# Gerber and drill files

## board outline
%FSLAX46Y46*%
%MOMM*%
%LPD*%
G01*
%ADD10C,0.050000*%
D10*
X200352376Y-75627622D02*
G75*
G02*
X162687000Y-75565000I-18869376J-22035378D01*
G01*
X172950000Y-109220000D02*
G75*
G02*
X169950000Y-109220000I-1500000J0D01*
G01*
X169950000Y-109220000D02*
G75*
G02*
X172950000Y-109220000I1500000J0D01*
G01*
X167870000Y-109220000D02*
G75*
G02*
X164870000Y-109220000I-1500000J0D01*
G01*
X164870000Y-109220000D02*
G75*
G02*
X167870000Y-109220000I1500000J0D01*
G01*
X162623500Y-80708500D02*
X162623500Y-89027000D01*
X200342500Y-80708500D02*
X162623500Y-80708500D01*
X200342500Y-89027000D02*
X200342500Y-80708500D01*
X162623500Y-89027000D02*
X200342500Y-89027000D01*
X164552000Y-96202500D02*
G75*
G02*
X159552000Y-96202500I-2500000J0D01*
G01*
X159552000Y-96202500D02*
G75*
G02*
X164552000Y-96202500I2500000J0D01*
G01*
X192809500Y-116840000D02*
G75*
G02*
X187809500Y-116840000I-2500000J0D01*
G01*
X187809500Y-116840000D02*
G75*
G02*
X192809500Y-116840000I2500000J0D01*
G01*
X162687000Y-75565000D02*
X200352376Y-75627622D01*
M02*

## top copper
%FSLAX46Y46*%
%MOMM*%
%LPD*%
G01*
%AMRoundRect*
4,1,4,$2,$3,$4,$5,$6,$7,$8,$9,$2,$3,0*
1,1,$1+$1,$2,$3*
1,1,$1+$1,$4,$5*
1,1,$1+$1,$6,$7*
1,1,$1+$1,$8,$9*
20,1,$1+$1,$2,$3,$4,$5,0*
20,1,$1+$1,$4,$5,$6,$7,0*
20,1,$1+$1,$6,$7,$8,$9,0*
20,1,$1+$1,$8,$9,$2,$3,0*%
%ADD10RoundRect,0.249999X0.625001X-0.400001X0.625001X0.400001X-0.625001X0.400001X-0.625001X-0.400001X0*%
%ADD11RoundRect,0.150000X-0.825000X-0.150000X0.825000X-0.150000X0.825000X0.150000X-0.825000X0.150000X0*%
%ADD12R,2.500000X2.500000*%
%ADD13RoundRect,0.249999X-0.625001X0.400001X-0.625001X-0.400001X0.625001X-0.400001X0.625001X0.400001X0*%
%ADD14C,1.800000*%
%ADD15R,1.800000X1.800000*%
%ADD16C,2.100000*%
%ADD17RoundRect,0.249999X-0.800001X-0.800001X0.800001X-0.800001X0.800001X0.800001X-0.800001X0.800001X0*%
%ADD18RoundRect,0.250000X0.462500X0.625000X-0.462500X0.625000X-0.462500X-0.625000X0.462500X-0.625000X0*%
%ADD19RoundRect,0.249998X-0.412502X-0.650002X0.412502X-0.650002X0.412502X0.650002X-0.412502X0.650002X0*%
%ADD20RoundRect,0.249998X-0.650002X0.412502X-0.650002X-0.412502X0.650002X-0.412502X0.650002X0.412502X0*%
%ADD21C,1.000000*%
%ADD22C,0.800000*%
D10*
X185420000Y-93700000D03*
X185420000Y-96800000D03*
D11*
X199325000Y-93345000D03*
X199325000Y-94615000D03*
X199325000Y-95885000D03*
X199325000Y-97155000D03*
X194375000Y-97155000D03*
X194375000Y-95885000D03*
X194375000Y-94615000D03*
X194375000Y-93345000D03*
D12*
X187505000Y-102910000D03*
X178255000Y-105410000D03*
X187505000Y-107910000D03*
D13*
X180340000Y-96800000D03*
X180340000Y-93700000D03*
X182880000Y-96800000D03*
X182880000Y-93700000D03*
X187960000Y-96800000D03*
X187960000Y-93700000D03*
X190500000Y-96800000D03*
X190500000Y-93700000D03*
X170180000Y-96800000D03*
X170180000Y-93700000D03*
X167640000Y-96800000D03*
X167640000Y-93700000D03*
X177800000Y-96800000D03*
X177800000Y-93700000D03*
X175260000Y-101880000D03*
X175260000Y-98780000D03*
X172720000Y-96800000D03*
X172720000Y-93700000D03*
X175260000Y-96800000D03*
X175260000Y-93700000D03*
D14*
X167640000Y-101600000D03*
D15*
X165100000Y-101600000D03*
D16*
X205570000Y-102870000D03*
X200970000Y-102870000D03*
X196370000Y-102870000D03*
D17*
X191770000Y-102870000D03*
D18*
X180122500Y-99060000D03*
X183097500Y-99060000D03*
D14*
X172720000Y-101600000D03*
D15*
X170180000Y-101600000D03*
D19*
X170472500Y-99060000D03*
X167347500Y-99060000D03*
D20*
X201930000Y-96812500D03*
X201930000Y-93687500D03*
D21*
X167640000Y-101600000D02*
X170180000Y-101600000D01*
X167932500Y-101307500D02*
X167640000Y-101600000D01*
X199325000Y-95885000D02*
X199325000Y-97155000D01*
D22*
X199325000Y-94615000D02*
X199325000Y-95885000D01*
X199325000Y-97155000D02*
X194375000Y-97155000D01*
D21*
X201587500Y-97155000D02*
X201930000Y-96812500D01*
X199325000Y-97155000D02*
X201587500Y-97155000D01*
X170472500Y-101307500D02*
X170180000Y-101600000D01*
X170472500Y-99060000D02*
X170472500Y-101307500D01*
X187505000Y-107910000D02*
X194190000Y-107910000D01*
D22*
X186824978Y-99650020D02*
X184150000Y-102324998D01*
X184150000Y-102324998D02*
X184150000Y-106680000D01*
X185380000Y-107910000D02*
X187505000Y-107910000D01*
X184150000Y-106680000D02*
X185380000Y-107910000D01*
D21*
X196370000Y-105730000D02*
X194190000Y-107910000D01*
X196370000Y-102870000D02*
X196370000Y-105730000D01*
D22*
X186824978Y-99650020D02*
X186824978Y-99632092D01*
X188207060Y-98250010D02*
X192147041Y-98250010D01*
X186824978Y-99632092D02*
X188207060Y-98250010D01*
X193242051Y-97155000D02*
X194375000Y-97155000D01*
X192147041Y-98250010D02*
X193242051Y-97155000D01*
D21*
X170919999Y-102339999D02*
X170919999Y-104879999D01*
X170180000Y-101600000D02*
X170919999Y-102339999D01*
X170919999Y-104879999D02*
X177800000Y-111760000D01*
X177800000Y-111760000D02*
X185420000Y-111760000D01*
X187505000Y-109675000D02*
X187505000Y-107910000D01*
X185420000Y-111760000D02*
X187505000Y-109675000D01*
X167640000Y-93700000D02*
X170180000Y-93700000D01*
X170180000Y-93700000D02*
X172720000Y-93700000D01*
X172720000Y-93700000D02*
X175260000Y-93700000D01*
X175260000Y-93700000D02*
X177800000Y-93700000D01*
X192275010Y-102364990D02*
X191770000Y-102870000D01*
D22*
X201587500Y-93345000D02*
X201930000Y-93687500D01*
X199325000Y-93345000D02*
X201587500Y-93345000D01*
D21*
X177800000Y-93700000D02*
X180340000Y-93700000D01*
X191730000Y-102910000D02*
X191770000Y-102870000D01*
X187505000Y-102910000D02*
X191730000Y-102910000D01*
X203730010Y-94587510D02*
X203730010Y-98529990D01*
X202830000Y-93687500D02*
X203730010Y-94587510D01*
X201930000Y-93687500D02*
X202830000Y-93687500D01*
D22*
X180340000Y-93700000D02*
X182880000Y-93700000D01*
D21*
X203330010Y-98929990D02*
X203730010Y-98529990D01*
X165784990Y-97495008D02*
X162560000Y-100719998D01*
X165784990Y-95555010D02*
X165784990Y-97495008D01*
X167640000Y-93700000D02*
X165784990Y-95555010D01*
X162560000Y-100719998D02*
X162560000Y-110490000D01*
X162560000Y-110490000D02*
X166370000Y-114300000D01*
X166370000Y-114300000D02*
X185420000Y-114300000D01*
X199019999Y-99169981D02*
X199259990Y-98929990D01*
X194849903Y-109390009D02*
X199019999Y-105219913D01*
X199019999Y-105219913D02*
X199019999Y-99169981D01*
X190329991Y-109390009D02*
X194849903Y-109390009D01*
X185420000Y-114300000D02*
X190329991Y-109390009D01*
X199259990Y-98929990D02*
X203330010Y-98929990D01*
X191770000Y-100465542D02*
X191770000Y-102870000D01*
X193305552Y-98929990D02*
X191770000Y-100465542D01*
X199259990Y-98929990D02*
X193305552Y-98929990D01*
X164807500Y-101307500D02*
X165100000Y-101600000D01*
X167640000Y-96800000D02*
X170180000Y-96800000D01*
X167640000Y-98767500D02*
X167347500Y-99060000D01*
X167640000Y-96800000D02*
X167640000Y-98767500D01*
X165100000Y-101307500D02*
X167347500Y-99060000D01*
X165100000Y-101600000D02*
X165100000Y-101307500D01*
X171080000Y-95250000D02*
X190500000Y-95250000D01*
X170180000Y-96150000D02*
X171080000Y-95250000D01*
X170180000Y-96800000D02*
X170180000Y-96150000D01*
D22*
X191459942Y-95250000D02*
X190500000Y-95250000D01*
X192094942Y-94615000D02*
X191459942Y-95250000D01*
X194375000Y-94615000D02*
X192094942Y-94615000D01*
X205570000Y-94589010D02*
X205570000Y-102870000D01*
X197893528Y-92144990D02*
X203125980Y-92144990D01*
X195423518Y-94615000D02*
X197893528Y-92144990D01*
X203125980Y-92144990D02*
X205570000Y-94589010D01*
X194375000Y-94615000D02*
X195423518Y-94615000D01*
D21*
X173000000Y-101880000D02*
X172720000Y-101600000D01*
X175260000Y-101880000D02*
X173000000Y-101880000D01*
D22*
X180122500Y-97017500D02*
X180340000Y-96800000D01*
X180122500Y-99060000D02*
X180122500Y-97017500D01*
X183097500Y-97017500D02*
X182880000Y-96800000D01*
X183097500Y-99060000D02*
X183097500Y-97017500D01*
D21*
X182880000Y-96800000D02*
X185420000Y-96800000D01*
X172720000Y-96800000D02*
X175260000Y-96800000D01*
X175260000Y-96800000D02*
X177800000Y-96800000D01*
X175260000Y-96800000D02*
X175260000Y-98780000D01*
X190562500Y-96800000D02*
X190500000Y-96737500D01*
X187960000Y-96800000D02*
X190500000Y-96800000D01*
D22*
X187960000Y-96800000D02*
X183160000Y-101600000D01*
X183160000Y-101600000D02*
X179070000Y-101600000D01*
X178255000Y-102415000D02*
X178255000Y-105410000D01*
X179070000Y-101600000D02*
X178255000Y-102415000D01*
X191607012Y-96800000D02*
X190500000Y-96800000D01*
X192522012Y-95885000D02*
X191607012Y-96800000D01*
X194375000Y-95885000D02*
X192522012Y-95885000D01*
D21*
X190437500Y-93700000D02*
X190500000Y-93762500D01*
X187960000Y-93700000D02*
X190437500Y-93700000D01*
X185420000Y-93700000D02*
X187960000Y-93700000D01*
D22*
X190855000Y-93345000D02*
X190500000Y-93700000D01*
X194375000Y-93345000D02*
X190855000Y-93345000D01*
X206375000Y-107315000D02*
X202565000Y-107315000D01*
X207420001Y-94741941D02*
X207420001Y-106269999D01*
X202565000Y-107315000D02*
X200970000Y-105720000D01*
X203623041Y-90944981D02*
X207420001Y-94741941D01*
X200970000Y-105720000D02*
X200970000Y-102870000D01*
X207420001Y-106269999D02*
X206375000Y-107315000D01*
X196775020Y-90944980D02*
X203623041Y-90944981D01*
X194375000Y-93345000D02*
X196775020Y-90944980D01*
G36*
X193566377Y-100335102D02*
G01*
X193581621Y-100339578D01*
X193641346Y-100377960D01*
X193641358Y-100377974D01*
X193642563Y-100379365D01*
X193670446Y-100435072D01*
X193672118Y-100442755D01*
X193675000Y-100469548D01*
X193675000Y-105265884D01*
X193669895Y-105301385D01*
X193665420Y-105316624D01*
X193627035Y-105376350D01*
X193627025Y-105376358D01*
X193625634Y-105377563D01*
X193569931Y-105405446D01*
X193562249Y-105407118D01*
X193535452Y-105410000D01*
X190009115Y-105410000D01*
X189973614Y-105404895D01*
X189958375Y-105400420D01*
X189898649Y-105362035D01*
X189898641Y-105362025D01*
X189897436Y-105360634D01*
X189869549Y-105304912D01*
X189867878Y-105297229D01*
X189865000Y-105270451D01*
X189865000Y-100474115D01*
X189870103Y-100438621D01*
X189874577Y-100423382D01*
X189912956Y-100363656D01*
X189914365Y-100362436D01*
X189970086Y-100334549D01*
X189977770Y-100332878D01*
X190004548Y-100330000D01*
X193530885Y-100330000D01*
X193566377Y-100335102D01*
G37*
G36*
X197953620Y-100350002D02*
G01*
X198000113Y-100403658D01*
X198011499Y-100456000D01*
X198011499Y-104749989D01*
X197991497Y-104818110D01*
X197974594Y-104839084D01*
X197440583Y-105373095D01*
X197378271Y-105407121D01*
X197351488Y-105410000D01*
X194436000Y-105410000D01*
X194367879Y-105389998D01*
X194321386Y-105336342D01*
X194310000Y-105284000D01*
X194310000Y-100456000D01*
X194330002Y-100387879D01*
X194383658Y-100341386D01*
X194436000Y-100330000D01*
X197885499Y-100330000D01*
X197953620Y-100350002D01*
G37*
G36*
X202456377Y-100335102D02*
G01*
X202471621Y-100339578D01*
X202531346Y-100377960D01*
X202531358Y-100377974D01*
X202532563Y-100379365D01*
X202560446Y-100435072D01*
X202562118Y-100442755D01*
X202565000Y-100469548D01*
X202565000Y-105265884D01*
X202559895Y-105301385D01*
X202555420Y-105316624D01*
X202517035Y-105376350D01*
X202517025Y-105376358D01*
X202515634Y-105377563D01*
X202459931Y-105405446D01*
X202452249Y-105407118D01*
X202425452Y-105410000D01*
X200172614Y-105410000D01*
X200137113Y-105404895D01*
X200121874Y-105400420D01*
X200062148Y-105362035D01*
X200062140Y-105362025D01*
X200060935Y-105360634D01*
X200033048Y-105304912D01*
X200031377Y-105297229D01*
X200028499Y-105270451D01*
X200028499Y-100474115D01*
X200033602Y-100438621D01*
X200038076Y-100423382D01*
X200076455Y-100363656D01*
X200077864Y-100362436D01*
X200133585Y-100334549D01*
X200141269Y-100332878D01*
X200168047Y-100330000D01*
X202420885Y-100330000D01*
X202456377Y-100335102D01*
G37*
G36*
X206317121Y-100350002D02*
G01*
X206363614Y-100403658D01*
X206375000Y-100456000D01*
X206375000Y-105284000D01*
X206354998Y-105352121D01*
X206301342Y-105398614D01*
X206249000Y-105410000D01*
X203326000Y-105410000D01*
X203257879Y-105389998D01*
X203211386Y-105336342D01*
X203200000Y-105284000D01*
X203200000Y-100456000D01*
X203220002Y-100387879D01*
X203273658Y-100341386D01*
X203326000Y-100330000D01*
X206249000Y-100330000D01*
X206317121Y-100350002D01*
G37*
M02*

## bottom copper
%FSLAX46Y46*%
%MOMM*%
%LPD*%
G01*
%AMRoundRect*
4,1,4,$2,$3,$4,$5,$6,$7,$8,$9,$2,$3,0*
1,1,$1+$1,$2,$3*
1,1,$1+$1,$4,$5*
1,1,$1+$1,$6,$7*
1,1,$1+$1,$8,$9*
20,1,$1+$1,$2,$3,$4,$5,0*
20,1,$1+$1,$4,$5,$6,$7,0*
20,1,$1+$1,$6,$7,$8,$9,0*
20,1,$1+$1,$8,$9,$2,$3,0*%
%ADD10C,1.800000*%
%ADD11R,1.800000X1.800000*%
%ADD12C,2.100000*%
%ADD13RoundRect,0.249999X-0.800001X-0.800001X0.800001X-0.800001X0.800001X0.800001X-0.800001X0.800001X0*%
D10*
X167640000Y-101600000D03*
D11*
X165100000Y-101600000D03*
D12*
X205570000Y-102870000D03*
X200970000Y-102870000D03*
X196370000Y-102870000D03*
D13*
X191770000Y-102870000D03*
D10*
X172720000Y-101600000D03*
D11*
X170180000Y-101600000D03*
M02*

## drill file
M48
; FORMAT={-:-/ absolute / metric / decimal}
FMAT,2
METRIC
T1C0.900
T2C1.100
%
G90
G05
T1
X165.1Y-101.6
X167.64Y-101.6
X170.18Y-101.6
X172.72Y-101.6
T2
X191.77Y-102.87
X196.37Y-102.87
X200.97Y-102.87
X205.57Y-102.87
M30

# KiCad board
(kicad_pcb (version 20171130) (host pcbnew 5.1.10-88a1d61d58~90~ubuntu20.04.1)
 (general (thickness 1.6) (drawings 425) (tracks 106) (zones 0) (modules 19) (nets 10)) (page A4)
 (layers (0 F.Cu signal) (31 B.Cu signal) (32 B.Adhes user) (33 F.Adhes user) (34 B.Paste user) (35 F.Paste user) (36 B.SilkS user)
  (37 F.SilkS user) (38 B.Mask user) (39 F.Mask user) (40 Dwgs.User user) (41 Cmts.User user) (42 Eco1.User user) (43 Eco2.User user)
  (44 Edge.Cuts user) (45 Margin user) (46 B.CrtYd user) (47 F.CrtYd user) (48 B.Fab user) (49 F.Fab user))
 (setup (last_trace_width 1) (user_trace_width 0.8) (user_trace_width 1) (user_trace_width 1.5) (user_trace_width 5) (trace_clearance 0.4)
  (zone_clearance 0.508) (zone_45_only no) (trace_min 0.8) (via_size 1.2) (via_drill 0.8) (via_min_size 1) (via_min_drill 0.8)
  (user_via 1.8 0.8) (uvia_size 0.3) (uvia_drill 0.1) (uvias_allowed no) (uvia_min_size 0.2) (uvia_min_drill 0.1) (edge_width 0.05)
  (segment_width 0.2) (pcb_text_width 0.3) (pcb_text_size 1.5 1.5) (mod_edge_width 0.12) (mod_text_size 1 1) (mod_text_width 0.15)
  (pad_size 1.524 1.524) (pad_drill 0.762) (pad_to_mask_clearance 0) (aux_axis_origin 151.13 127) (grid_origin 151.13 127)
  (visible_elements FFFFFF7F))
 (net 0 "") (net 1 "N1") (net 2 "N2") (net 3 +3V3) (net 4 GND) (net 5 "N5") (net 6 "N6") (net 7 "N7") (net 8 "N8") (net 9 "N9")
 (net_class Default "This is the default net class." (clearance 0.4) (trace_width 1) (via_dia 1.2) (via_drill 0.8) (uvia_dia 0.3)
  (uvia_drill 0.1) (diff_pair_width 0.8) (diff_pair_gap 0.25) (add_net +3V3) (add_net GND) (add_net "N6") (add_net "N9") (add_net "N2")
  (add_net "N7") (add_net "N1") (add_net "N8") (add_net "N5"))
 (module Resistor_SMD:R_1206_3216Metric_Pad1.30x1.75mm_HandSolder (layer F.Cu) (at 185.42 95.25 90)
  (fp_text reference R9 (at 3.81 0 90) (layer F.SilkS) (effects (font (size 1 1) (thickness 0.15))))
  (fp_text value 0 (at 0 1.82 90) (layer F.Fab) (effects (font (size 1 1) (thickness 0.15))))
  (pad 2 smd roundrect (at 1.55 0 90) (size 1.3 1.75) (layers F.Cu F.Paste F.Mask) (roundrect_rratio 0.1923069230769231) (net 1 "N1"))
  (pad 1 smd roundrect (at -1.55 0 90) (size 1.3 1.75) (layers F.Cu F.Paste F.Mask) (roundrect_rratio 0.1923069230769231) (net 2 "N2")))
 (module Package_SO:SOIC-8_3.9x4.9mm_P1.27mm (layer F.Cu) (at 196.85 95.25)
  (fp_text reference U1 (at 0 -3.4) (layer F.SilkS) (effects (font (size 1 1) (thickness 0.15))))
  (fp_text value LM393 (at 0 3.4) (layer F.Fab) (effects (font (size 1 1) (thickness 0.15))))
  (pad 8 smd roundrect (at 2.475 -1.905) (size 1.95 0.6) (layers F.Cu F.Paste F.Mask) (roundrect_rratio 0.25) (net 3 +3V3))
  (pad 7 smd roundrect (at 2.475 -0.635) (size 1.95 0.6) (layers F.Cu F.Paste F.Mask) (roundrect_rratio 0.25) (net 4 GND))
  (pad 6 smd roundrect (at 2.475 0.635) (size 1.95 0.6) (layers F.Cu F.Paste F.Mask) (roundrect_rratio 0.25) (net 4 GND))
  (pad 5 smd roundrect (at 2.475 1.905) (size 1.95 0.6) (layers F.Cu F.Paste F.Mask) (roundrect_rratio 0.25) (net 4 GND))
  (pad 4 smd roundrect (at -2.475 1.905) (size 1.95 0.6) (layers F.Cu F.Paste F.Mask) (roundrect_rratio 0.25) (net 4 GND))
  (pad 3 smd roundrect (at -2.475 0.635) (size 1.95 0.6) (layers F.Cu F.Paste F.Mask) (roundrect_rratio 0.25) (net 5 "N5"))
  (pad 2 smd roundrect (at -2.475 -0.635) (size 1.95 0.6) (layers F.Cu F.Paste F.Mask) (roundrect_rratio 0.25) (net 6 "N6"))
  (pad 1 smd roundrect (at -2.475 -1.905) (size 1.95 0.6) (layers F.Cu F.Paste F.Mask) (roundrect_rratio 0.25) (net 1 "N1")))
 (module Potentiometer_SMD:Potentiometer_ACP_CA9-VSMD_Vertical (layer F.Cu) (at 182.88 105.41 180)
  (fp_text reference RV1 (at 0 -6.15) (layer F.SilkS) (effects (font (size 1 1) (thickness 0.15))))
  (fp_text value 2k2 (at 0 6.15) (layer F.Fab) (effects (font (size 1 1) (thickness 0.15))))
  (pad 1 smd rect (at -4.625 2.5 180) (size 2.5 2.5) (layers F.Cu F.Paste F.Mask) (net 3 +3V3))
  (pad 2 smd rect (at 4.625 0 180) (size 2.5 2.5) (layers F.Cu F.Paste F.Mask) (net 5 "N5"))
  (pad 3 smd rect (at -4.625 -2.5 180) (size 2.5 2.5) (layers F.Cu F.Paste F.Mask) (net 4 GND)))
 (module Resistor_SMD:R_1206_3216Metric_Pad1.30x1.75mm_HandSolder (layer F.Cu) (at 180.34 95.25 270)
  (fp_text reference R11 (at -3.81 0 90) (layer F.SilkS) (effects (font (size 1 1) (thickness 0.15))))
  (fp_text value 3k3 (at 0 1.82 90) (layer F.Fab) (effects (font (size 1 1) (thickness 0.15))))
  (pad 2 smd roundrect (at 1.55 0 270) (size 1.3 1.75) (layers F.Cu F.Paste F.Mask) (roundrect_rratio 0.1923069230769231) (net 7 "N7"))
  (pad 1 smd roundrect (at -1.55 0 270) (size 1.3 1.75) (layers F.Cu F.Paste F.Mask) (roundrect_rratio 0.1923069230769231) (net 3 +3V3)))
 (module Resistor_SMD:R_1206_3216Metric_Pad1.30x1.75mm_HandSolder (layer F.Cu) (at 182.88 95.25 270)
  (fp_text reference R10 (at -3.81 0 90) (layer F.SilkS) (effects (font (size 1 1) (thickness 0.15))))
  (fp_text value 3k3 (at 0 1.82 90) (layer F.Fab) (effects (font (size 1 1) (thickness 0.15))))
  (pad 2 smd roundrect (at 1.55 0 270) (size 1.3 1.75) (layers F.Cu F.Paste F.Mask) (roundrect_rratio 0.1923069230769231) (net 2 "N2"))
  (pad 1 smd roundrect (at -1.55 0 270) (size 1.3 1.75) (layers F.Cu F.Paste F.Mask) (roundrect_rratio 0.1923069230769231) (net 3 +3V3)))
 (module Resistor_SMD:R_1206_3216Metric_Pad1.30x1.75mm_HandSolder (layer F.Cu) (at 187.96 95.25 270)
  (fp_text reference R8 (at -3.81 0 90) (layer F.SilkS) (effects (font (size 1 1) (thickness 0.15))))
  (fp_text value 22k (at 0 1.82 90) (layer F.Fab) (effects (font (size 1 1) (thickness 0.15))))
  (pad 2 smd roundrect (at 1.55 0 270) (size 1.3 1.75) (layers F.Cu F.Paste F.Mask) (roundrect_rratio 0.1923069230769231) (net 5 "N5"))
  (pad 1 smd roundrect (at -1.55 0 270) (size 1.3 1.75) (layers F.Cu F.Paste F.Mask) (roundrect_rratio 0.1923069230769231) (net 1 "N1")))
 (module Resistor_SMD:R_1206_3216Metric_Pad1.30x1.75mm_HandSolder (layer F.Cu) (at 190.5 95.25 270)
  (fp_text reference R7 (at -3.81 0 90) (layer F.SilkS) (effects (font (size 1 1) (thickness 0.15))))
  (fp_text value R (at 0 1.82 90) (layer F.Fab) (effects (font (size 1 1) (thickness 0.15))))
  (pad 2 smd roundrect (at 1.55 0 270) (size 1.3 1.75) (layers F.Cu F.Paste F.Mask) (roundrect_rratio 0.1923069230769231) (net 5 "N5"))
  (pad 1 smd roundrect (at -1.55 0 270) (size 1.3 1.75) (layers F.Cu F.Paste F.Mask) (roundrect_rratio 0.1923069230769231) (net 1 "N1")))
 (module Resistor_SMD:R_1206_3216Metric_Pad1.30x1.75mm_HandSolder (layer F.Cu) (at 170.18 95.25 270)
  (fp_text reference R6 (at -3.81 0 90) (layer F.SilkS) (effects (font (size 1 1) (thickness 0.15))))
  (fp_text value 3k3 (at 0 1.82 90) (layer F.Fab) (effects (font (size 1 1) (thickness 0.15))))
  (pad 2 smd roundrect (at 1.55 0 270) (size 1.3 1.75) (layers F.Cu F.Paste F.Mask) (roundrect_rratio 0.1923069230769231) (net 6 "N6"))
  (pad 1 smd roundrect (at -1.55 0 270) (size 1.3 1.75) (layers F.Cu F.Paste F.Mask) (roundrect_rratio 0.1923069230769231) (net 3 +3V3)))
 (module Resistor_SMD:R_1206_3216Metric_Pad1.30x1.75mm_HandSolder (layer F.Cu) (at 167.64 95.25 270)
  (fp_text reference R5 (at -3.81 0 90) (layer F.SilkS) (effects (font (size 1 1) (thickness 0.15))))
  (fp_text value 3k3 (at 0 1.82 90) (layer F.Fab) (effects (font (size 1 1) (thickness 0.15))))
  (pad 2 smd roundrect (at 1.55 0 270) (size 1.3 1.75) (layers F.Cu F.Paste F.Mask) (roundrect_rratio 0.1923069230769231) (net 6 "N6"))
  (pad 1 smd roundrect (at -1.55 0 270) (size 1.3 1.75) (layers F.Cu F.Paste F.Mask) (roundrect_rratio 0.1923069230769231) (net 3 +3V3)))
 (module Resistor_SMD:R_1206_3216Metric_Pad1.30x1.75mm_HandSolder (layer F.Cu) (at 177.8 95.25 270)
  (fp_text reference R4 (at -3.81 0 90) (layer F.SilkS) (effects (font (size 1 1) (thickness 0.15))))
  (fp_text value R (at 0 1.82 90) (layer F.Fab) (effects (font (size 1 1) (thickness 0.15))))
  (pad 2 smd roundrect (at 1.55 0 270) (size 1.3 1.75) (layers F.Cu F.Paste F.Mask) (roundrect_rratio 0.1923069230769231) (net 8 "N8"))
  (pad 1 smd roundrect (at -1.55 0 270) (size 1.3 1.75) (layers F.Cu F.Paste F.Mask) (roundrect_rratio 0.1923069230769231) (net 3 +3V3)))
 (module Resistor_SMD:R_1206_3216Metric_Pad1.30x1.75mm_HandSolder (layer F.Cu) (at 175.26 100.33 270)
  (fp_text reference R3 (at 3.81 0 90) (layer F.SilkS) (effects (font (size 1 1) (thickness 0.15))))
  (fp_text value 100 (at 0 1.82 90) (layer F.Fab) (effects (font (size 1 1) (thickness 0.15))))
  (pad 2 smd roundrect (at 1.55 0 270) (size 1.3 1.75) (layers F.Cu F.Paste F.Mask) (roundrect_rratio 0.1923069230769231) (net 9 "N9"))
  (pad 1 smd roundrect (at -1.55 0 270) (size 1.3 1.75) (layers F.Cu F.Paste F.Mask) (roundrect_rratio 0.1923069230769231) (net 8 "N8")))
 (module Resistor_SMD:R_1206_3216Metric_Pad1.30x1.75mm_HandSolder (layer F.Cu) (at 172.72 95.25 270)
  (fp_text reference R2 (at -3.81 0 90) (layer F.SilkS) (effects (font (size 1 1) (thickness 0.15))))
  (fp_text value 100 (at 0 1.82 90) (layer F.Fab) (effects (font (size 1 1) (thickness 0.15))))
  (pad 2 smd roundrect (at 1.55 0 270) (size 1.3 1.75) (layers F.Cu F.Paste F.Mask) (roundrect_rratio 0.1923069230769231) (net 8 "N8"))
  (pad 1 smd roundrect (at -1.55 0 270) (size 1.3 1.75) (layers F.Cu F.Paste F.Mask) (roundrect_rratio 0.1923069230769231) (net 3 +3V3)))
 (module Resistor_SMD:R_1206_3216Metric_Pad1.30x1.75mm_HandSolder (layer F.Cu) (at 175.26 95.25 270)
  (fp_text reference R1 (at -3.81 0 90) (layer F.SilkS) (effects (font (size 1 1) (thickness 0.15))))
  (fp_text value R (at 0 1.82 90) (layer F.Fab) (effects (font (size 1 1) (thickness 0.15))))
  (pad 2 smd roundrect (at 1.55 0 270) (size 1.3 1.75) (layers F.Cu F.Paste F.Mask) (roundrect_rratio 0.1923069230769231) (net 8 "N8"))
  (pad 1 smd roundrect (at -1.55 0 270) (size 1.3 1.75) (layers F.Cu F.Paste F.Mask) (roundrect_rratio 0.1923069230769231) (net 3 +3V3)))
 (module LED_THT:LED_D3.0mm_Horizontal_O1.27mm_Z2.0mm (layer F.Cu) (at 165.1 101.6)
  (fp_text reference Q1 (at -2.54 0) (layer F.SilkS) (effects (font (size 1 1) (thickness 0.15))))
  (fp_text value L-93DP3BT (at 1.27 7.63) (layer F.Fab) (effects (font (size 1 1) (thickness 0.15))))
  (pad 2 thru_hole circle (at 2.54 0) (size 1.8 1.8) (drill 0.9) (layers *.Cu *.Mask) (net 4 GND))
  (pad 1 thru_hole rect (at 0 0) (size 1.8 1.8) (drill 0.9) (layers *.Cu *.Mask) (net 6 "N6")))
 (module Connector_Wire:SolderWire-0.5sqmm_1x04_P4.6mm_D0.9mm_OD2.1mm (layer F.Cu) (at 191.77 102.87)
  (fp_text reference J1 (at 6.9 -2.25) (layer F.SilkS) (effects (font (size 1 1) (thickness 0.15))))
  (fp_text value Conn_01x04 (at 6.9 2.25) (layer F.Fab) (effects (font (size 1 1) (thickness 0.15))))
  (pad 4 thru_hole circle (at 13.8 0) (size 2.1 2.1) (drill 1.1) (layers *.Cu *.Mask) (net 6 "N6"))
  (pad 3 thru_hole circle (at 9.2 0) (size 2.1 2.1) (drill 1.1) (layers *.Cu *.Mask) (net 1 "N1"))
  (pad 2 thru_hole circle (at 4.6 0) (size 2.1 2.1) (drill 1.1) (layers *.Cu *.Mask) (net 4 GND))
  (pad 1 thru_hole roundrect (at 0 0) (size 2.1 2.1) (drill 1.1) (layers *.Cu *.Mask) (roundrect_rratio 0.1190471428571429) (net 3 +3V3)))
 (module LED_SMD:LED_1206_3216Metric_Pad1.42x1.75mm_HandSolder (layer F.Cu) (at 181.61 99.06 180)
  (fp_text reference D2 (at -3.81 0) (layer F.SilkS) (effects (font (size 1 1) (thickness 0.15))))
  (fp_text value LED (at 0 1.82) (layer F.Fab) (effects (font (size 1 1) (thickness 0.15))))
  (pad 2 smd roundrect (at 1.4875 0 180) (size 1.425 1.75) (layers F.Cu F.Paste F.Mask) (roundrect_rratio 0.1754385964912281) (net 7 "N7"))
  (pad 1 smd roundrect (at -1.4875 0 180) (size 1.425 1.75) (layers F.Cu F.Paste F.Mask) (roundrect_rratio 0.1754385964912281) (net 2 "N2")))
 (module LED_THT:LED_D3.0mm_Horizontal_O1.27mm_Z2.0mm (layer F.Cu) (at 170.18 101.6)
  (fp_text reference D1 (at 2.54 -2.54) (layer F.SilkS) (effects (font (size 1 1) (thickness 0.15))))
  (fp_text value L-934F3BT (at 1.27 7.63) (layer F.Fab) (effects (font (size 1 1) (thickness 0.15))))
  (pad 2 thru_hole circle (at 2.54 0) (size 1.8 1.8) (drill 0.9) (layers *.Cu *.Mask) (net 9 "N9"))
  (pad 1 thru_hole rect (at 0 0) (size 1.8 1.8) (drill 0.9) (layers *.Cu *.Mask) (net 4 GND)))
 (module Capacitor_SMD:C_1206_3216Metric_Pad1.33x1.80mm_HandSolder (layer F.Cu) (at 168.91 99.06)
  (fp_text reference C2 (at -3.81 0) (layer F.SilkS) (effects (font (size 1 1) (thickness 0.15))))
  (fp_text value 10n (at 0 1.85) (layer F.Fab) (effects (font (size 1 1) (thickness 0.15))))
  (pad 2 smd roundrect (at 1.5625 0) (size 1.325 1.8) (layers F.Cu F.Paste F.Mask) (roundrect_rratio 0.1886777358490566) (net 4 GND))
  (pad 1 smd roundrect (at -1.5625 0) (size 1.325 1.8) (layers F.Cu F.Paste F.Mask) (roundrect_rratio 0.1886777358490566) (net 6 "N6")))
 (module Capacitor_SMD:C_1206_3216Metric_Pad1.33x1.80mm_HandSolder (layer F.Cu) (at 201.93 95.25 270)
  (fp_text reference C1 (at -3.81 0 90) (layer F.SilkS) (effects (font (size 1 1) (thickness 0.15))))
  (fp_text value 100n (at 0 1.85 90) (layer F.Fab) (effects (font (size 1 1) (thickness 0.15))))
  (pad 2 smd roundrect (at 1.5625 0 270) (size 1.325 1.8) (layers F.Cu F.Paste F.Mask) (roundrect_rratio 0.1886777358490566) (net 4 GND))
  (pad 1 smd roundrect (at -1.5625 0 270) (size 1.325 1.8) (layers F.Cu F.Paste F.Mask) (roundrect_rratio 0.1886777358490566) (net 3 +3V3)))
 (gr_arc (start 181.483 97.663) (end 162.687 75.565) (angle -279.0421861) (layer Edge.Cuts) (width 0.05))
 (gr_circle (center 171.45 109.22) (end 172.95 109.22) (layer Edge.Cuts) (width 0.05))
 (gr_circle (center 166.37 109.22) (end 167.87 109.22) (layer Edge.Cuts) (width 0.05))
 (gr_line (start 162.6235 80.7085) (end 162.6235 89.027) (layer Edge.Cuts) (width 0.05))
 (gr_line (start 200.3425 80.7085) (end 162.6235 80.7085) (layer Edge.Cuts) (width 0.05))
 (gr_line (start 200.3425 89.027) (end 200.3425 80.7085) (layer Edge.Cuts) (width 0.05))
 (gr_line (start 162.6235 89.027) (end 200.3425 89.027) (layer Edge.Cuts) (width 0.05))
 (gr_circle (center 162.052 96.2025) (end 164.552 96.2025) (layer Edge.Cuts) (width 0.05))
 (gr_circle (center 190.3095 116.84) (end 192.8095 116.84) (layer Edge.Cuts) (width 0.05))
 (gr_line (start 162.687 75.565) (end 200.352376 75.627622) (layer Edge.Cuts) (width 0.05))
 (segment (start 167.64 101.6) (end 170.18 101.6) (width 1) (layer F.Cu) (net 4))
 (segment (start 167.9325 101.3075) (end 167.64 101.6) (width 1) (layer F.Cu) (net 4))
 (segment (start 199.325 95.885) (end 199.325 97.155) (width 1) (layer F.Cu) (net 4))
 (segment (start 199.325 94.615) (end 199.325 95.885) (width 0.8) (layer F.Cu) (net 4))
 (segment (start 199.325 97.155) (end 194.375 97.155) (width 0.8) (layer F.Cu) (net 4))
 (segment (start 201.5875 97.155) (end 201.93 96.8125) (width 1) (layer F.Cu) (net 4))
 (segment (start 199.325 97.155) (end 201.5875 97.155) (width 1) (layer F.Cu) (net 4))
 (segment (start 170.4725 101.3075) (end 170.18 101.6) (width 1) (layer F.Cu) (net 4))
 (segment (start 170.4725 99.06) (end 170.4725 101.3075) (width 1) (layer F.Cu) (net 4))
 (segment (start 187.505 107.91) (end 194.19 107.91) (width 1) (layer F.Cu) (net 4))
 (segment (start 186.824978 99.65002) (end 184.15 102.324998) (width 0.8) (layer F.Cu) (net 4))
 (segment (start 184.15 102.324998) (end 184.15 106.68) (width 0.8) (layer F.Cu) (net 4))
 (segment (start 185.38 107.91) (end 187.505 107.91) (width 0.8) (layer F.Cu) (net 4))
 (segment (start 184.15 106.68) (end 185.38 107.91) (width 0.8) (layer F.Cu) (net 4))
 (segment (start 196.37 105.73) (end 194.19 107.91) (width 1) (layer F.Cu) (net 4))
 (segment (start 196.37 102.87) (end 196.37 105.73) (width 1) (layer F.Cu) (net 4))
 (segment (start 186.824978 99.65002) (end 186.824978 99.632092) (width 0.8) (layer F.Cu) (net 4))
 (segment (start 188.20706 98.25001) (end 192.147041 98.25001) (width 0.8) (layer F.Cu) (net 4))
 (segment (start 186.824978 99.632092) (end 188.20706 98.25001) (width 0.8) (layer F.Cu) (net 4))
 (segment (start 193.242051 97.155) (end 194.375 97.155) (width 0.8) (layer F.Cu) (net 4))
 (segment (start 192.147041 98.25001) (end 193.242051 97.155) (width 0.8) (layer F.Cu) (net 4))
 (segment (start 170.919999 102.339999) (end 170.919999 104.879999) (width 1) (layer F.Cu) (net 4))
 (segment (start 170.18 101.6) (end 170.919999 102.339999) (width 1) (layer F.Cu) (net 4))
 (segment (start 170.919999 104.879999) (end 177.8 111.76) (width 1) (layer F.Cu) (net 4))
 (segment (start 177.8 111.76) (end 185.42 111.76) (width 1) (layer F.Cu) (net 4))
 (segment (start 187.505 109.675) (end 187.505 107.91) (width 1) (layer F.Cu) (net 4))
 (segment (start 185.42 111.76) (end 187.505 109.675) (width 1) (layer F.Cu) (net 4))
 (segment (start 167.64 93.7) (end 170.18 93.7) (width 1) (layer F.Cu) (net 3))
 (segment (start 170.18 93.7) (end 172.72 93.7) (width 1) (layer F.Cu) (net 3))
 (segment (start 172.72 93.7) (end 175.26 93.7) (width 1) (layer F.Cu) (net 3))
 (segment (start 175.26 93.7) (end 177.8 93.7) (width 1) (layer F.Cu) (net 3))
 (segment (start 192.27501 102.36499) (end 191.77 102.87) (width 1) (layer F.Cu) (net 3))
 (segment (start 201.5875 93.345) (end 201.93 93.6875) (width 0.8) (layer F.Cu) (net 3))
 (segment (start 199.325 93.345) (end 201.5875 93.345) (width 0.8) (layer F.Cu) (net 3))
 (segment (start 177.8 93.7) (end 180.34 93.7) (width 1) (layer F.Cu) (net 3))
 (segment (start 191.73 102.91) (end 191.77 102.87) (width 1) (layer F.Cu) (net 3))
 (segment (start 187.505 102.91) (end 191.73 102.91) (width 1) (layer F.Cu) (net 3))
 (segment (start 203.73001 94.58751) (end 203.73001 98.52999) (width 1) (layer F.Cu) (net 3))
 (segment (start 202.83 93.6875) (end 203.73001 94.58751) (width 1) (layer F.Cu) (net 3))
 (segment (start 201.93 93.6875) (end 202.83 93.6875) (width 1) (layer F.Cu) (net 3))
 (segment (start 180.34 93.7) (end 182.88 93.7) (width 0.8) (layer F.Cu) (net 3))
 (segment (start 203.33001 98.92999) (end 203.73001 98.52999) (width 1) (layer F.Cu) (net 3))
 (segment (start 165.78499 97.495008) (end 162.56 100.719998) (width 1) (layer F.Cu) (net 3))
 (segment (start 165.78499 95.55501) (end 165.78499 97.495008) (width 1) (layer F.Cu) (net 3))
 (segment (start 167.64 93.7) (end 165.78499 95.55501) (width 1) (layer F.Cu) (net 3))
 (segment (start 162.56 100.719998) (end 162.56 110.49) (width 1) (layer F.Cu) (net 3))
 (segment (start 162.56 110.49) (end 166.37 114.3) (width 1) (layer F.Cu) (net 3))
 (segment (start 166.37 114.3) (end 185.42 114.3) (width 1) (layer F.Cu) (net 3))
 (segment (start 199.019999 99.169981) (end 199.25999 98.92999) (width 1) (layer F.Cu) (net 3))
 (segment (start 194.849903 109.390009) (end 199.019999 105.219913) (width 1) (layer F.Cu) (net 3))
 (segment (start 199.019999 105.219913) (end 199.019999 99.169981) (width 1) (layer F.Cu) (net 3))
 (segment (start 190.329991 109.390009) (end 194.849903 109.390009) (width 1) (layer F.Cu) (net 3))
 (segment (start 185.42 114.3) (end 190.329991 109.390009) (width 1) (layer F.Cu) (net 3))
 (segment (start 199.25999 98.92999) (end 203.33001 98.92999) (width 1) (layer F.Cu) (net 3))
 (segment (start 191.77 100.465542) (end 191.77 102.87) (width 1) (layer F.Cu) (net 3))
 (segment (start 193.305552 98.92999) (end 191.77 100.465542) (width 1) (layer F.Cu) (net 3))
 (segment (start 199.25999 98.92999) (end 193.305552 98.92999) (width 1) (layer F.Cu) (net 3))
 (segment (start 164.8075 101.3075) (end 165.1 101.6) (width 1) (layer F.Cu) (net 6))
 (segment (start 167.64 96.8) (end 170.18 96.8) (width 1) (layer F.Cu) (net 6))
 (segment (start 167.64 98.7675) (end 167.3475 99.06) (width 1) (layer F.Cu) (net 6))
 (segment (start 167.64 96.8) (end 167.64 98.7675) (width 1) (layer F.Cu) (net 6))
 (segment (start 165.1 101.3075) (end 167.3475 99.06) (width 1) (layer F.Cu) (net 6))
 (segment (start 165.1 101.6) (end 165.1 101.3075) (width 1) (layer F.Cu) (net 6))
 (segment (start 171.08 95.25) (end 190.5 95.25) (width 1) (layer F.Cu) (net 6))
 (segment (start 170.18 96.15) (end 171.08 95.25) (width 1) (layer F.Cu) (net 6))
 (segment (start 170.18 96.8) (end 170.18 96.15) (width 1) (layer F.Cu) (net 6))
 (segment (start 191.459942 95.25) (end 190.5 95.25) (width 0.8) (layer F.Cu) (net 6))
 (segment (start 192.094942 94.615) (end 191.459942 95.25) (width 0.8) (layer F.Cu) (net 6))
 (segment (start 194.375 94.615) (end 192.094942 94.615) (width 0.8) (layer F.Cu) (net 6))
 (segment (start 205.57 94.58901) (end 205.57 102.87) (width 0.8) (layer F.Cu) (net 6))
 (segment (start 197.893528 92.14499) (end 203.12598 92.14499) (width 0.8) (layer F.Cu) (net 6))
 (segment (start 195.423518 94.615) (end 197.893528 92.14499) (width 0.8) (layer F.Cu) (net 6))
 (segment (start 203.12598 92.14499) (end 205.57 94.58901) (width 0.8) (layer F.Cu) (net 6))
 (segment (start 194.375 94.615) (end 195.423518 94.615) (width 0.8) (layer F.Cu) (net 6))
 (segment (start 173 101.88) (end 172.72 101.6) (width 1) (layer F.Cu) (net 9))
 (segment (start 175.26 101.88) (end 173 101.88) (width 1) (layer F.Cu) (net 9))
 (segment (start 180.1225 97.0175) (end 180.34 96.8) (width 0.8) (layer F.Cu) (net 7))
 (segment (start 180.1225 99.06) (end 180.1225 97.0175) (width 0.8) (layer F.Cu) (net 7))
 (segment (start 183.0975 97.0175) (end 182.88 96.8) (width 0.8) (layer F.Cu) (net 2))
 (segment (start 183.0975 99.06) (end 183.0975 97.0175) (width 0.8) (layer F.Cu) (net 2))
 (segment (start 182.88 96.8) (end 185.42 96.8) (width 1) (layer F.Cu) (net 2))
 (segment (start 172.72 96.8) (end 175.26 96.8) (width 1) (layer F.Cu) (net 8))
 (segment (start 175.26 96.8) (end 177.8 96.8) (width 1) (layer F.Cu) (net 8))
 (segment (start 175.26 96.8) (end 175.26 98.78) (width 1) (layer F.Cu) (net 8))
 (segment (start 190.5625 96.8) (end 190.5 96.7375) (width 1) (layer F.Cu) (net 5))
 (segment (start 187.96 96.8) (end 190.5 96.8) (width 1) (layer F.Cu) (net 5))
 (segment (start 187.96 96.8) (end 183.16 101.6) (width 0.8) (layer F.Cu) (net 5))
 (segment (start 183.16 101.6) (end 179.07 101.6) (width 0.8) (layer F.Cu) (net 5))
 (segment (start 178.255 102.415) (end 178.255 105.41) (width 0.8) (layer F.Cu) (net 5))
 (segment (start 179.07 101.6) (end 178.255 102.415) (width 0.8) (layer F.Cu) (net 5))
 (segment (start 191.607012 96.8) (end 190.5 96.8) (width 0.8) (layer F.Cu) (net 5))
 (segment (start 192.522012 95.885) (end 191.607012 96.8) (width 0.8) (layer F.Cu) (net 5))
 (segment (start 194.375 95.885) (end 192.522012 95.885) (width 0.8) (layer F.Cu) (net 5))
 (segment (start 190.4375 93.7) (end 190.5 93.7625) (width 1) (layer F.Cu) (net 1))
 (segment (start 187.96 93.7) (end 190.4375 93.7) (width 1) (layer F.Cu) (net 1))
 (segment (start 185.42 93.7) (end 187.96 93.7) (width 1) (layer F.Cu) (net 1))
 (segment (start 190.855 93.345) (end 190.5 93.7) (width 0.8) (layer F.Cu) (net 1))
 (segment (start 194.375 93.345) (end 190.855 93.345) (width 0.8) (layer F.Cu) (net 1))
 (segment (start 206.375 107.315) (end 202.565 107.315) (width 0.8) (layer F.Cu) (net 1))
 (segment (start 207.420001 94.741941) (end 207.420001 106.269999) (width 0.8) (layer F.Cu) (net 1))
 (segment (start 202.565 107.315) (end 200.97 105.72) (width 0.8) (layer F.Cu) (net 1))
 (segment (start 203.623041 90.944981) (end 207.420001 94.741941) (width 0.8) (layer F.Cu) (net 1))
 (segment (start 200.97 105.72) (end 200.97 102.87) (width 0.8) (layer F.Cu) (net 1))
 (segment (start 207.420001 106.269999) (end 206.375 107.315) (width 0.8) (layer F.Cu) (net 1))
 (segment (start 196.77502 90.94498) (end 203.623041 90.944981) (width 0.8) (layer F.Cu) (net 1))
 (segment (start 194.375 93.345) (end 196.77502 90.94498) (width 0.8) (layer F.Cu) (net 1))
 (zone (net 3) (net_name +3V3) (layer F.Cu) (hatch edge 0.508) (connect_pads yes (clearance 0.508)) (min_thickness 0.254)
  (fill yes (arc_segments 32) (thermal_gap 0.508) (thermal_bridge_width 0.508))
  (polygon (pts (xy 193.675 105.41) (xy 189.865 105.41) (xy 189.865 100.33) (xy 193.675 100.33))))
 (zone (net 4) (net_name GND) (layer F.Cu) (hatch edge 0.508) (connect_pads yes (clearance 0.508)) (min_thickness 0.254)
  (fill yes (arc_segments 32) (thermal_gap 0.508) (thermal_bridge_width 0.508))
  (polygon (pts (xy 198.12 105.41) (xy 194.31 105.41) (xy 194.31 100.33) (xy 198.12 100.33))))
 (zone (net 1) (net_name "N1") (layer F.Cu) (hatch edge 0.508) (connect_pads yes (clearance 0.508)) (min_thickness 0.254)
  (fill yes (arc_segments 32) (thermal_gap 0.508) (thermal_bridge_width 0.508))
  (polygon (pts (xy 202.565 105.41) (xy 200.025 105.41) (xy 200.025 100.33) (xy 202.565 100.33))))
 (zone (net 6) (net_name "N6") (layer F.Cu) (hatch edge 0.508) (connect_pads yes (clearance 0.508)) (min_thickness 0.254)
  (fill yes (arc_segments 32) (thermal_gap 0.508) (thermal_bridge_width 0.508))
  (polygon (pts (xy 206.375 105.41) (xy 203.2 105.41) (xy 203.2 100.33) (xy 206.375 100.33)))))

